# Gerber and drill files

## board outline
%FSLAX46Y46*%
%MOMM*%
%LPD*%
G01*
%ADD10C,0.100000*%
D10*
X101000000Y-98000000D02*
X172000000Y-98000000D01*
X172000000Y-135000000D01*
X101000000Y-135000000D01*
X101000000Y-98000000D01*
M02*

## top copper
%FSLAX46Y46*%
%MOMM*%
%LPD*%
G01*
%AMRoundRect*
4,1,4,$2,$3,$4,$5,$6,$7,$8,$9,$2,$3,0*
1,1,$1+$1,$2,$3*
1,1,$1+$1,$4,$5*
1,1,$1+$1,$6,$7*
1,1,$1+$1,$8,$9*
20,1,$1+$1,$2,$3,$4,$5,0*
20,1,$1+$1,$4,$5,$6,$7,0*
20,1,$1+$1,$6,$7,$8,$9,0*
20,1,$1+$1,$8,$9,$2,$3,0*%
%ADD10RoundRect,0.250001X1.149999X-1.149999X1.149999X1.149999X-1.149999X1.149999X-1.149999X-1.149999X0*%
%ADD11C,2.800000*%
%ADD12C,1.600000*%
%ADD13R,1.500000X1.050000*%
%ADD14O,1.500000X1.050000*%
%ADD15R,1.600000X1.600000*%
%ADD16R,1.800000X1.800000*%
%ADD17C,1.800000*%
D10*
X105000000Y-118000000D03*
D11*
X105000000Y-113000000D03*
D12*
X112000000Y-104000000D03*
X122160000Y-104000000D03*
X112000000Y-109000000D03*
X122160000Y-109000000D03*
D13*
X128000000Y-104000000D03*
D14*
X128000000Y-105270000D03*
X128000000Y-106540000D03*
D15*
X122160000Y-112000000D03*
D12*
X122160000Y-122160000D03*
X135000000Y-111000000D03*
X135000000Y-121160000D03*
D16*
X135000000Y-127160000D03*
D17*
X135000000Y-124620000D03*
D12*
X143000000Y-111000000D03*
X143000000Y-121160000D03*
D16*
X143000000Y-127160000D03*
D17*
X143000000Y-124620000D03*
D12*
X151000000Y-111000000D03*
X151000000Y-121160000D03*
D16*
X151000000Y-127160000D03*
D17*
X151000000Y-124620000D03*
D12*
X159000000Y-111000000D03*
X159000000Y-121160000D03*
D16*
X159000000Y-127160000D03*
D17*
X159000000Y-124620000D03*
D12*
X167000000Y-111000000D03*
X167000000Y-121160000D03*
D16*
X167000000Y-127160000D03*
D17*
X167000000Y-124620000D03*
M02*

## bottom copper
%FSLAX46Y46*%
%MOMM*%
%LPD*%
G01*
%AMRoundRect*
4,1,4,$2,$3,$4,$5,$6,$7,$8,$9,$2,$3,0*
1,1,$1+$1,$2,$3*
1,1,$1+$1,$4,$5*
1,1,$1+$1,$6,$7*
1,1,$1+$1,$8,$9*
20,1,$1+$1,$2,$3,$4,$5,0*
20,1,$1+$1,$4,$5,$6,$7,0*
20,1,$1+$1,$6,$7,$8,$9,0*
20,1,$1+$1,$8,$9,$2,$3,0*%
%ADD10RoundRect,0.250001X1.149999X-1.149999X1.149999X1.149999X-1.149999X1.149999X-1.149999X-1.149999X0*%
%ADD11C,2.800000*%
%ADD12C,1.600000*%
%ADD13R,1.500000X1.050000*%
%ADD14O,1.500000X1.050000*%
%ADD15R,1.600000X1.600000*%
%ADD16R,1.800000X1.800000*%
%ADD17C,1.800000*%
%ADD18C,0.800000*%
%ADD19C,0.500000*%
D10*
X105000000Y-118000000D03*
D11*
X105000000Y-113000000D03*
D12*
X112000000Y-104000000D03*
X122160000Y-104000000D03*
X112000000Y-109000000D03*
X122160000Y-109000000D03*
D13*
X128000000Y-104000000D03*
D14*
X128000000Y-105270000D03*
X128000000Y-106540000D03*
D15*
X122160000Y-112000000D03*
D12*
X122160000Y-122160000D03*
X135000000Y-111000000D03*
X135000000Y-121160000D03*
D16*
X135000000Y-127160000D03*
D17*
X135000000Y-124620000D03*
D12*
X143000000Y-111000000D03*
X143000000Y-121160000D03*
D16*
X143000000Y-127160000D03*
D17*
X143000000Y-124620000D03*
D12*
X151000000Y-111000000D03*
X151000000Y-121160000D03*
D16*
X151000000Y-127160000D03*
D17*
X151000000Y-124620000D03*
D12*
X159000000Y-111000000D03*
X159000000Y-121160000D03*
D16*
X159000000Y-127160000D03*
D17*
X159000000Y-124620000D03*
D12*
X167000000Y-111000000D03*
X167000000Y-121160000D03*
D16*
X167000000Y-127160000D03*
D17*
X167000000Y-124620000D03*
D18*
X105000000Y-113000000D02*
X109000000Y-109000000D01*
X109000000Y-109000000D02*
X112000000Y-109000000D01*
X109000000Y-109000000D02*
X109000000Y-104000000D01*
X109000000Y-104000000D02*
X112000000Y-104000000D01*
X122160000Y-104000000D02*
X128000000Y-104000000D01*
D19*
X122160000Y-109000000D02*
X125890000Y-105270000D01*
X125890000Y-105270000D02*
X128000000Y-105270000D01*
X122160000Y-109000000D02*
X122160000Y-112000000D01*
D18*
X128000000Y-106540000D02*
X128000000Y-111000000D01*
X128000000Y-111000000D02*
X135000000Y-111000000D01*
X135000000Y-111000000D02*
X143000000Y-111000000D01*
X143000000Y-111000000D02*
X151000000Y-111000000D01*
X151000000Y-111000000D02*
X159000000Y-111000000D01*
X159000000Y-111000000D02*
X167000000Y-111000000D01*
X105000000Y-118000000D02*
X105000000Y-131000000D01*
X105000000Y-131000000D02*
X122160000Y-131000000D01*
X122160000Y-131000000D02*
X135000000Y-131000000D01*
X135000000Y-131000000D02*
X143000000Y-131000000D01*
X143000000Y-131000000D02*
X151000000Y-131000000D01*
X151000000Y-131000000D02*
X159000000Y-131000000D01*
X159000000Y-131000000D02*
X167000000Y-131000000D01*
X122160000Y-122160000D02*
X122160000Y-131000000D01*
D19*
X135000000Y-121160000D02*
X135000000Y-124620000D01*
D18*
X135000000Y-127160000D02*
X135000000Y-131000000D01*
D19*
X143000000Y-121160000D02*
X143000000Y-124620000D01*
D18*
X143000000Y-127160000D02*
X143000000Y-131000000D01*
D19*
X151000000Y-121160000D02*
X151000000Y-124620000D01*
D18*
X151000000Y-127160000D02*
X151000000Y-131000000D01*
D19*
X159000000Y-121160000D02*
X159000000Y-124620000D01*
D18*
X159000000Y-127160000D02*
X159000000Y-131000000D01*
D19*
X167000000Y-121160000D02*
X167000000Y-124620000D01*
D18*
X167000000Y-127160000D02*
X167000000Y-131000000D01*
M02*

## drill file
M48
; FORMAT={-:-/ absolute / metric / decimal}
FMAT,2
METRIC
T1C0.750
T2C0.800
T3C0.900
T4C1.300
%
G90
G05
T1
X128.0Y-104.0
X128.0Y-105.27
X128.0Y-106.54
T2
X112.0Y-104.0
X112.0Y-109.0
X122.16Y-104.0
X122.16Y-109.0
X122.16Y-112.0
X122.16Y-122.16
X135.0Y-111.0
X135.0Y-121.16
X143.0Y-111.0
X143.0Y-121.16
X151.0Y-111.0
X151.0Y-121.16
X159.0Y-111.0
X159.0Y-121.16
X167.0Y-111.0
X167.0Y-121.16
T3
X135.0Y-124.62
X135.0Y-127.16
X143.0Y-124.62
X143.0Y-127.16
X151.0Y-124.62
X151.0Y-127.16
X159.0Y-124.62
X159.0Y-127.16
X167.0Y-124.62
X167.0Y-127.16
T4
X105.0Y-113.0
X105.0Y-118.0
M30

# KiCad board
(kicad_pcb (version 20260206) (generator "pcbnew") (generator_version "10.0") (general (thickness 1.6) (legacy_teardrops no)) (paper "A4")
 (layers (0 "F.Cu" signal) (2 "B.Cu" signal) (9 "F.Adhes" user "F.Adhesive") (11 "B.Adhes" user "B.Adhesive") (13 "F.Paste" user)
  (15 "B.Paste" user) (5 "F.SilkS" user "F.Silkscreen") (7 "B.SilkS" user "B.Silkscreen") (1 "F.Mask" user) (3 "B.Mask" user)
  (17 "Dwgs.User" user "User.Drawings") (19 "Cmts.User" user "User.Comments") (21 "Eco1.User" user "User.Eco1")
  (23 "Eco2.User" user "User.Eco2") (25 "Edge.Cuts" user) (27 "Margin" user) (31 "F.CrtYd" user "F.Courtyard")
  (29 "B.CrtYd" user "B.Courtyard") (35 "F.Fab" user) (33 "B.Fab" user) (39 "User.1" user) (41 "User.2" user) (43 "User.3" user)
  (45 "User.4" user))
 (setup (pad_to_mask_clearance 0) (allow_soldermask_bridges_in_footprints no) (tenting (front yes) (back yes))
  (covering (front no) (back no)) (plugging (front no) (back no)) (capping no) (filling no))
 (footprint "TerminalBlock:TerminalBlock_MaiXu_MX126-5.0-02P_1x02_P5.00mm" (layer "F.Cu") (at 105 118 90)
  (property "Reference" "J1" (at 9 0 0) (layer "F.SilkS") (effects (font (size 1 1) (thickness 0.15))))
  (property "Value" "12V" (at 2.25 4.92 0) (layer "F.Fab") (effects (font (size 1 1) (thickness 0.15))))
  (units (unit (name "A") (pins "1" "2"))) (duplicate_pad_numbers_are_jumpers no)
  (pad "1" thru_hole roundrect (at 0 0 90) (size 2.8 2.8) (drill 1.3) (layers "*.Cu" "*.Mask") (remove_unused_layers no)
   (roundrect_rratio 0.089286) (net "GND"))
  (pad "2" thru_hole circle (at 5 0 90) (size 2.8 2.8) (drill 1.3) (layers "*.Cu" "*.Mask") (remove_unused_layers no) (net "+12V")))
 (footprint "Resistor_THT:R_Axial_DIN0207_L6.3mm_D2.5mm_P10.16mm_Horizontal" (layer "F.Cu") (at 112 104)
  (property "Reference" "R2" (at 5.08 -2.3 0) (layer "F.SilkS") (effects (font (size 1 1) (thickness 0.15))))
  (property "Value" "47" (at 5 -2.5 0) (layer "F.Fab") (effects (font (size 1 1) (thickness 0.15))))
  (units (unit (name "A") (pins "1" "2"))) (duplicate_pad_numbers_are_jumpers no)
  (pad "1" thru_hole circle (at 0 0) (size 1.6 1.6) (drill 0.8) (layers "*.Cu" "*.Mask") (remove_unused_layers no) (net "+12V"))
  (pad "2" thru_hole circle (at 10.16 0) (size 1.6 1.6) (drill 0.8) (layers "*.Cu" "*.Mask") (remove_unused_layers no) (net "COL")))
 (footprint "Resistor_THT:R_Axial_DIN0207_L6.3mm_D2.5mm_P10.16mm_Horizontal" (layer "F.Cu") (at 112 109)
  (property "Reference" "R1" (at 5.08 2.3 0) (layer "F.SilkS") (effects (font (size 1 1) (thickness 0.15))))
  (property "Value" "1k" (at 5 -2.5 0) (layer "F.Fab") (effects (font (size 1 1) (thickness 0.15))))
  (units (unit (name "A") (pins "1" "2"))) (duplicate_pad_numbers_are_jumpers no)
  (pad "1" thru_hole circle (at 0 0) (size 1.6 1.6) (drill 0.8) (layers "*.Cu" "*.Mask") (remove_unused_layers no) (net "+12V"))
  (pad "2" thru_hole circle (at 10.16 0) (size 1.6 1.6) (drill 0.8) (layers "*.Cu" "*.Mask") (remove_unused_layers no) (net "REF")))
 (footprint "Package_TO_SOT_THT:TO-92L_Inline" (layer "F.Cu") (at 128 104 -90)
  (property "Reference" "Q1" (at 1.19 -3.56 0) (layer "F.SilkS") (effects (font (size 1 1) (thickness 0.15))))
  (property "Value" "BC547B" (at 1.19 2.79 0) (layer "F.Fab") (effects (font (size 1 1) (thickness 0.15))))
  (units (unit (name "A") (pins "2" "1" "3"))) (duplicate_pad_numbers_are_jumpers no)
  (pad "1" thru_hole rect (at 0 0 270) (size 1.05 1.5) (drill 0.75) (layers "*.Cu" "*.Mask") (remove_unused_layers no) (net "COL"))
  (pad "2" thru_hole oval (at 1.27 0 270) (size 1.05 1.5) (drill 0.75) (layers "*.Cu" "*.Mask") (remove_unused_layers no) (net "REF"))
  (pad "3" thru_hole oval (at 2.54 0 270) (size 1.05 1.5) (drill 0.75) (layers "*.Cu" "*.Mask") (remove_unused_layers no) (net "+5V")))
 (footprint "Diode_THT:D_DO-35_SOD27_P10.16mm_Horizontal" (layer "F.Cu") (at 122.16 112 -90)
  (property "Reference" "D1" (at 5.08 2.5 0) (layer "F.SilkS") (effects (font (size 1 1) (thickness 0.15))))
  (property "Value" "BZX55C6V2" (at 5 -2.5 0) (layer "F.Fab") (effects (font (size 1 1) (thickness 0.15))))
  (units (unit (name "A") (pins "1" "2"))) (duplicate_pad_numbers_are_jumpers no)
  (pad "1" thru_hole rect (at 0 0 270) (size 1.6 1.6) (drill 0.8) (layers "*.Cu" "*.Mask") (remove_unused_layers no) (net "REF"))
  (pad "2" thru_hole circle (at 10.16 0 270) (size 1.6 1.6) (drill 0.8) (layers "*.Cu" "*.Mask") (remove_unused_layers no) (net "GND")))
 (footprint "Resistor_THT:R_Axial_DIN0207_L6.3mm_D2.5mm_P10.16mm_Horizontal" (layer "F.Cu") (at 135 111 -90)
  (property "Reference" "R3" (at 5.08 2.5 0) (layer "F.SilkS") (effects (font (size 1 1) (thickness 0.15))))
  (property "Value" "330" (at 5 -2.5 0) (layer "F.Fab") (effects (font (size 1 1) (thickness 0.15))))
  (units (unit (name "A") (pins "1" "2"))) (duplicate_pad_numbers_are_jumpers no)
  (pad "1" thru_hole circle (at 0 0 270) (size 1.6 1.6) (drill 0.8) (layers "*.Cu" "*.Mask") (remove_unused_layers no) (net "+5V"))
  (pad "2" thru_hole circle (at 10.16 0 270) (size 1.6 1.6) (drill 0.8) (layers "*.Cu" "*.Mask") (remove_unused_layers no) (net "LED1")))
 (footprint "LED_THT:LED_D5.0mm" (layer "F.Cu") (at 135 127.16 90)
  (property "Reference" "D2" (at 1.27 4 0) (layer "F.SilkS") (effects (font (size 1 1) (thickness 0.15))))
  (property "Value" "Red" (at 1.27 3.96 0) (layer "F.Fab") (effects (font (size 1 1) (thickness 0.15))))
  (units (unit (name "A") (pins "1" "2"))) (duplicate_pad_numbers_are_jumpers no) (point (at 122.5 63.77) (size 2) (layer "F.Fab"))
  (pad "1" thru_hole rect (at 0 0 90) (size 1.8 1.8) (drill 0.9) (layers "*.Cu" "*.Mask") (remove_unused_layers no) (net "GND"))
  (pad "2" thru_hole circle (at 2.54 0 90) (size 1.8 1.8) (drill 0.9) (layers "*.Cu" "*.Mask") (remove_unused_layers no) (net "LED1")))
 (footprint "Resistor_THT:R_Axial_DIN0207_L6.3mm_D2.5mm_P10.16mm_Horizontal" (layer "F.Cu") (at 143 111 -90)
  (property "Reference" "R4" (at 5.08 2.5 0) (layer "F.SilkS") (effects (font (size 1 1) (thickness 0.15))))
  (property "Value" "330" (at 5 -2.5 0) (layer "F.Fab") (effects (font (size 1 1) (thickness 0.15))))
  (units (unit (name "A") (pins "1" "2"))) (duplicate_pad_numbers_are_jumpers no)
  (pad "1" thru_hole circle (at 0 0 270) (size 1.6 1.6) (drill 0.8) (layers "*.Cu" "*.Mask") (remove_unused_layers no) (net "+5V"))
  (pad "2" thru_hole circle (at 10.16 0 270) (size 1.6 1.6) (drill 0.8) (layers "*.Cu" "*.Mask") (remove_unused_layers no) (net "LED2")))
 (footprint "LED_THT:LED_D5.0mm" (layer "F.Cu") (at 143 127.16 90)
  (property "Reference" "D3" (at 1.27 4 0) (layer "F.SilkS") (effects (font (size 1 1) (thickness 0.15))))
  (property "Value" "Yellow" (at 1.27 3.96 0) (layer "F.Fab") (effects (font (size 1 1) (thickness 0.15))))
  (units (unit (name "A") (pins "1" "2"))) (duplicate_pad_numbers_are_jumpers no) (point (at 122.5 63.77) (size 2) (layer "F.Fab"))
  (pad "1" thru_hole rect (at 0 0 90) (size 1.8 1.8) (drill 0.9) (layers "*.Cu" "*.Mask") (remove_unused_layers no) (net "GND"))
  (pad "2" thru_hole circle (at 2.54 0 90) (size 1.8 1.8) (drill 0.9) (layers "*.Cu" "*.Mask") (remove_unused_layers no) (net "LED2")))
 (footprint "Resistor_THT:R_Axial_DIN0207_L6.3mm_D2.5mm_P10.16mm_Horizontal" (layer "F.Cu") (at 151 111 -90)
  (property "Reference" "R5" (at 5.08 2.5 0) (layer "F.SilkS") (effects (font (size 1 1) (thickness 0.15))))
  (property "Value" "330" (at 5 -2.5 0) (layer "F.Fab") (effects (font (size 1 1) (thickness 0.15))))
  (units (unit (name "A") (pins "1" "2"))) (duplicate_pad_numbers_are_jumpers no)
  (pad "1" thru_hole circle (at 0 0 270) (size 1.6 1.6) (drill 0.8) (layers "*.Cu" "*.Mask") (remove_unused_layers no) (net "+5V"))
  (pad "2" thru_hole circle (at 10.16 0 270) (size 1.6 1.6) (drill 0.8) (layers "*.Cu" "*.Mask") (remove_unused_layers no) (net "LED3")))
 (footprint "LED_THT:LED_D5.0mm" (layer "F.Cu") (at 151 127.16 90)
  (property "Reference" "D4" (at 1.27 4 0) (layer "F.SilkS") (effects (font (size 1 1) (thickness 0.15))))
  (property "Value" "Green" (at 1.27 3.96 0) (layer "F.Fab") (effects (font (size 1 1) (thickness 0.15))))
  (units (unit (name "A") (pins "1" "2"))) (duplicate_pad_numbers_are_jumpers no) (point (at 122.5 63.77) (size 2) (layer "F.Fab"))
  (pad "1" thru_hole rect (at 0 0 90) (size 1.8 1.8) (drill 0.9) (layers "*.Cu" "*.Mask") (remove_unused_layers no) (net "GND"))
  (pad "2" thru_hole circle (at 2.54 0 90) (size 1.8 1.8) (drill 0.9) (layers "*.Cu" "*.Mask") (remove_unused_layers no) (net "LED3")))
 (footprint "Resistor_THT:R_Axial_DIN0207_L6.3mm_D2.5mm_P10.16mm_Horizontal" (layer "F.Cu") (at 159 111 -90)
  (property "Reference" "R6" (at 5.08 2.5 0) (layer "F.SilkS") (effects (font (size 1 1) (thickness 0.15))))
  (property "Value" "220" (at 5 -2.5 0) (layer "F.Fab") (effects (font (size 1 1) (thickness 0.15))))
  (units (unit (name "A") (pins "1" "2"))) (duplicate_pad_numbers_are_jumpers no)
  (pad "1" thru_hole circle (at 0 0 270) (size 1.6 1.6) (drill 0.8) (layers "*.Cu" "*.Mask") (remove_unused_layers no) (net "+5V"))
  (pad "2" thru_hole circle (at 10.16 0 270) (size 1.6 1.6) (drill 0.8) (layers "*.Cu" "*.Mask") (remove_unused_layers no) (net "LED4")))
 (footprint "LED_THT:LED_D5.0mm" (layer "F.Cu") (at 159 127.16 90)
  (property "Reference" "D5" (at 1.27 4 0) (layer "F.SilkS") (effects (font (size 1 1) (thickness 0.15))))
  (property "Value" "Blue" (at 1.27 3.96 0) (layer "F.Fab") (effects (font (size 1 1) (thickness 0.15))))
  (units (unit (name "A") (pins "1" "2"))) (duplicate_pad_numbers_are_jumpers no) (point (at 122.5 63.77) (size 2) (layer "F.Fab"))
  (pad "1" thru_hole rect (at 0 0 90) (size 1.8 1.8) (drill 0.9) (layers "*.Cu" "*.Mask") (remove_unused_layers no) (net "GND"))
  (pad "2" thru_hole circle (at 2.54 0 90) (size 1.8 1.8) (drill 0.9) (layers "*.Cu" "*.Mask") (remove_unused_layers no) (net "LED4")))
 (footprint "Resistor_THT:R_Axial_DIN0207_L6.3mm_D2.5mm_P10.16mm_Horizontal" (layer "F.Cu") (at 167 111 -90)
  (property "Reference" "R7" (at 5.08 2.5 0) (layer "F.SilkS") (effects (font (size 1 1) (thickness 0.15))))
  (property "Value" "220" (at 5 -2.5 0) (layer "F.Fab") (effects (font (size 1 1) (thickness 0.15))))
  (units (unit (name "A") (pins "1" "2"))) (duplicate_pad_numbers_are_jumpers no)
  (pad "1" thru_hole circle (at 0 0 270) (size 1.6 1.6) (drill 0.8) (layers "*.Cu" "*.Mask") (remove_unused_layers no) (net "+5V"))
  (pad "2" thru_hole circle (at 10.16 0 270) (size 1.6 1.6) (drill 0.8) (layers "*.Cu" "*.Mask") (remove_unused_layers no) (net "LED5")))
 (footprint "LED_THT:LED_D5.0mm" (layer "F.Cu") (at 167 127.16 90)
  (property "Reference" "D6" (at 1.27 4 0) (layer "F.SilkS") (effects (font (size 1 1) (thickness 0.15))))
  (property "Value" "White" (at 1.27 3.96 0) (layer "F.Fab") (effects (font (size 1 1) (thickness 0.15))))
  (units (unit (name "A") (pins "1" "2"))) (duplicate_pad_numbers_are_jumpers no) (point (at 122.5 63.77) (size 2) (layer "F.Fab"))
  (pad "1" thru_hole rect (at 0 0 90) (size 1.8 1.8) (drill 0.9) (layers "*.Cu" "*.Mask") (remove_unused_layers no) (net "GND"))
  (pad "2" thru_hole circle (at 2.54 0 90) (size 1.8 1.8) (drill 0.9) (layers "*.Cu" "*.Mask") (remove_unused_layers no) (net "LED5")))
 (gr_rect (start 101 98) (end 172 135) (stroke (width 0.1) (type default)) (fill no) (layer "Edge.Cuts"))
 (segment (start 105 113) (end 109 109) (width 0.8) (layer "B.Cu") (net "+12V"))
 (segment (start 109 109) (end 112 109) (width 0.8) (layer "B.Cu") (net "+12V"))
 (segment (start 109 109) (end 109 104) (width 0.8) (layer "B.Cu") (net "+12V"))
 (segment (start 109 104) (end 112 104) (width 0.8) (layer "B.Cu") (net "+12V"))
 (segment (start 122.16 104) (end 128 104) (width 0.8) (layer "B.Cu") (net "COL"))
 (segment (start 122.16 109) (end 125.89 105.27) (width 0.5) (layer "B.Cu") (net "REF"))
 (segment (start 125.89 105.27) (end 128 105.27) (width 0.5) (layer "B.Cu") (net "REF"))
 (segment (start 122.16 109) (end 122.16 112) (width 0.5) (layer "B.Cu") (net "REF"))
 (segment (start 128 106.54) (end 128 111) (width 0.8) (layer "B.Cu") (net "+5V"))
 (segment (start 128 111) (end 135 111) (width 0.8) (layer "B.Cu") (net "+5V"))
 (segment (start 135 111) (end 143 111) (width 0.8) (layer "B.Cu") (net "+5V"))
 (segment (start 143 111) (end 151 111) (width 0.8) (layer "B.Cu") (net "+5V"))
 (segment (start 151 111) (end 159 111) (width 0.8) (layer "B.Cu") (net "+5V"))
 (segment (start 159 111) (end 167 111) (width 0.8) (layer "B.Cu") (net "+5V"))
 (segment (start 105 118) (end 105 131) (width 0.8) (layer "B.Cu") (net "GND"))
 (segment (start 105 131) (end 122.16 131) (width 0.8) (layer "B.Cu") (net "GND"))
 (segment (start 122.16 131) (end 135 131) (width 0.8) (layer "B.Cu") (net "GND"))
 (segment (start 135 131) (end 143 131) (width 0.8) (layer "B.Cu") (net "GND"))
 (segment (start 143 131) (end 151 131) (width 0.8) (layer "B.Cu") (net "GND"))
 (segment (start 151 131) (end 159 131) (width 0.8) (layer "B.Cu") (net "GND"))
 (segment (start 159 131) (end 167 131) (width 0.8) (layer "B.Cu") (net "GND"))
 (segment (start 122.16 122.16) (end 122.16 131) (width 0.8) (layer "B.Cu") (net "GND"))
 (segment (start 135 121.16) (end 135 124.62) (width 0.5) (layer "B.Cu") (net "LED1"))
 (segment (start 135 127.16) (end 135 131) (width 0.8) (layer "B.Cu") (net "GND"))
 (segment (start 143 121.16) (end 143 124.62) (width 0.5) (layer "B.Cu") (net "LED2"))
 (segment (start 143 127.16) (end 143 131) (width 0.8) (layer "B.Cu") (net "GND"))
 (segment (start 151 121.16) (end 151 124.62) (width 0.5) (layer "B.Cu") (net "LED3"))
 (segment (start 151 127.16) (end 151 131) (width 0.8) (layer "B.Cu") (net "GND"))
 (segment (start 159 121.16) (end 159 124.62) (width 0.5) (layer "B.Cu") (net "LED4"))
 (segment (start 159 127.16) (end 159 131) (width 0.8) (layer "B.Cu") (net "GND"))
 (segment (start 167 121.16) (end 167 124.62) (width 0.5) (layer "B.Cu") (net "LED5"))
 (segment (start 167 127.16) (end 167 131) (width 0.8) (layer "B.Cu") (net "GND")))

